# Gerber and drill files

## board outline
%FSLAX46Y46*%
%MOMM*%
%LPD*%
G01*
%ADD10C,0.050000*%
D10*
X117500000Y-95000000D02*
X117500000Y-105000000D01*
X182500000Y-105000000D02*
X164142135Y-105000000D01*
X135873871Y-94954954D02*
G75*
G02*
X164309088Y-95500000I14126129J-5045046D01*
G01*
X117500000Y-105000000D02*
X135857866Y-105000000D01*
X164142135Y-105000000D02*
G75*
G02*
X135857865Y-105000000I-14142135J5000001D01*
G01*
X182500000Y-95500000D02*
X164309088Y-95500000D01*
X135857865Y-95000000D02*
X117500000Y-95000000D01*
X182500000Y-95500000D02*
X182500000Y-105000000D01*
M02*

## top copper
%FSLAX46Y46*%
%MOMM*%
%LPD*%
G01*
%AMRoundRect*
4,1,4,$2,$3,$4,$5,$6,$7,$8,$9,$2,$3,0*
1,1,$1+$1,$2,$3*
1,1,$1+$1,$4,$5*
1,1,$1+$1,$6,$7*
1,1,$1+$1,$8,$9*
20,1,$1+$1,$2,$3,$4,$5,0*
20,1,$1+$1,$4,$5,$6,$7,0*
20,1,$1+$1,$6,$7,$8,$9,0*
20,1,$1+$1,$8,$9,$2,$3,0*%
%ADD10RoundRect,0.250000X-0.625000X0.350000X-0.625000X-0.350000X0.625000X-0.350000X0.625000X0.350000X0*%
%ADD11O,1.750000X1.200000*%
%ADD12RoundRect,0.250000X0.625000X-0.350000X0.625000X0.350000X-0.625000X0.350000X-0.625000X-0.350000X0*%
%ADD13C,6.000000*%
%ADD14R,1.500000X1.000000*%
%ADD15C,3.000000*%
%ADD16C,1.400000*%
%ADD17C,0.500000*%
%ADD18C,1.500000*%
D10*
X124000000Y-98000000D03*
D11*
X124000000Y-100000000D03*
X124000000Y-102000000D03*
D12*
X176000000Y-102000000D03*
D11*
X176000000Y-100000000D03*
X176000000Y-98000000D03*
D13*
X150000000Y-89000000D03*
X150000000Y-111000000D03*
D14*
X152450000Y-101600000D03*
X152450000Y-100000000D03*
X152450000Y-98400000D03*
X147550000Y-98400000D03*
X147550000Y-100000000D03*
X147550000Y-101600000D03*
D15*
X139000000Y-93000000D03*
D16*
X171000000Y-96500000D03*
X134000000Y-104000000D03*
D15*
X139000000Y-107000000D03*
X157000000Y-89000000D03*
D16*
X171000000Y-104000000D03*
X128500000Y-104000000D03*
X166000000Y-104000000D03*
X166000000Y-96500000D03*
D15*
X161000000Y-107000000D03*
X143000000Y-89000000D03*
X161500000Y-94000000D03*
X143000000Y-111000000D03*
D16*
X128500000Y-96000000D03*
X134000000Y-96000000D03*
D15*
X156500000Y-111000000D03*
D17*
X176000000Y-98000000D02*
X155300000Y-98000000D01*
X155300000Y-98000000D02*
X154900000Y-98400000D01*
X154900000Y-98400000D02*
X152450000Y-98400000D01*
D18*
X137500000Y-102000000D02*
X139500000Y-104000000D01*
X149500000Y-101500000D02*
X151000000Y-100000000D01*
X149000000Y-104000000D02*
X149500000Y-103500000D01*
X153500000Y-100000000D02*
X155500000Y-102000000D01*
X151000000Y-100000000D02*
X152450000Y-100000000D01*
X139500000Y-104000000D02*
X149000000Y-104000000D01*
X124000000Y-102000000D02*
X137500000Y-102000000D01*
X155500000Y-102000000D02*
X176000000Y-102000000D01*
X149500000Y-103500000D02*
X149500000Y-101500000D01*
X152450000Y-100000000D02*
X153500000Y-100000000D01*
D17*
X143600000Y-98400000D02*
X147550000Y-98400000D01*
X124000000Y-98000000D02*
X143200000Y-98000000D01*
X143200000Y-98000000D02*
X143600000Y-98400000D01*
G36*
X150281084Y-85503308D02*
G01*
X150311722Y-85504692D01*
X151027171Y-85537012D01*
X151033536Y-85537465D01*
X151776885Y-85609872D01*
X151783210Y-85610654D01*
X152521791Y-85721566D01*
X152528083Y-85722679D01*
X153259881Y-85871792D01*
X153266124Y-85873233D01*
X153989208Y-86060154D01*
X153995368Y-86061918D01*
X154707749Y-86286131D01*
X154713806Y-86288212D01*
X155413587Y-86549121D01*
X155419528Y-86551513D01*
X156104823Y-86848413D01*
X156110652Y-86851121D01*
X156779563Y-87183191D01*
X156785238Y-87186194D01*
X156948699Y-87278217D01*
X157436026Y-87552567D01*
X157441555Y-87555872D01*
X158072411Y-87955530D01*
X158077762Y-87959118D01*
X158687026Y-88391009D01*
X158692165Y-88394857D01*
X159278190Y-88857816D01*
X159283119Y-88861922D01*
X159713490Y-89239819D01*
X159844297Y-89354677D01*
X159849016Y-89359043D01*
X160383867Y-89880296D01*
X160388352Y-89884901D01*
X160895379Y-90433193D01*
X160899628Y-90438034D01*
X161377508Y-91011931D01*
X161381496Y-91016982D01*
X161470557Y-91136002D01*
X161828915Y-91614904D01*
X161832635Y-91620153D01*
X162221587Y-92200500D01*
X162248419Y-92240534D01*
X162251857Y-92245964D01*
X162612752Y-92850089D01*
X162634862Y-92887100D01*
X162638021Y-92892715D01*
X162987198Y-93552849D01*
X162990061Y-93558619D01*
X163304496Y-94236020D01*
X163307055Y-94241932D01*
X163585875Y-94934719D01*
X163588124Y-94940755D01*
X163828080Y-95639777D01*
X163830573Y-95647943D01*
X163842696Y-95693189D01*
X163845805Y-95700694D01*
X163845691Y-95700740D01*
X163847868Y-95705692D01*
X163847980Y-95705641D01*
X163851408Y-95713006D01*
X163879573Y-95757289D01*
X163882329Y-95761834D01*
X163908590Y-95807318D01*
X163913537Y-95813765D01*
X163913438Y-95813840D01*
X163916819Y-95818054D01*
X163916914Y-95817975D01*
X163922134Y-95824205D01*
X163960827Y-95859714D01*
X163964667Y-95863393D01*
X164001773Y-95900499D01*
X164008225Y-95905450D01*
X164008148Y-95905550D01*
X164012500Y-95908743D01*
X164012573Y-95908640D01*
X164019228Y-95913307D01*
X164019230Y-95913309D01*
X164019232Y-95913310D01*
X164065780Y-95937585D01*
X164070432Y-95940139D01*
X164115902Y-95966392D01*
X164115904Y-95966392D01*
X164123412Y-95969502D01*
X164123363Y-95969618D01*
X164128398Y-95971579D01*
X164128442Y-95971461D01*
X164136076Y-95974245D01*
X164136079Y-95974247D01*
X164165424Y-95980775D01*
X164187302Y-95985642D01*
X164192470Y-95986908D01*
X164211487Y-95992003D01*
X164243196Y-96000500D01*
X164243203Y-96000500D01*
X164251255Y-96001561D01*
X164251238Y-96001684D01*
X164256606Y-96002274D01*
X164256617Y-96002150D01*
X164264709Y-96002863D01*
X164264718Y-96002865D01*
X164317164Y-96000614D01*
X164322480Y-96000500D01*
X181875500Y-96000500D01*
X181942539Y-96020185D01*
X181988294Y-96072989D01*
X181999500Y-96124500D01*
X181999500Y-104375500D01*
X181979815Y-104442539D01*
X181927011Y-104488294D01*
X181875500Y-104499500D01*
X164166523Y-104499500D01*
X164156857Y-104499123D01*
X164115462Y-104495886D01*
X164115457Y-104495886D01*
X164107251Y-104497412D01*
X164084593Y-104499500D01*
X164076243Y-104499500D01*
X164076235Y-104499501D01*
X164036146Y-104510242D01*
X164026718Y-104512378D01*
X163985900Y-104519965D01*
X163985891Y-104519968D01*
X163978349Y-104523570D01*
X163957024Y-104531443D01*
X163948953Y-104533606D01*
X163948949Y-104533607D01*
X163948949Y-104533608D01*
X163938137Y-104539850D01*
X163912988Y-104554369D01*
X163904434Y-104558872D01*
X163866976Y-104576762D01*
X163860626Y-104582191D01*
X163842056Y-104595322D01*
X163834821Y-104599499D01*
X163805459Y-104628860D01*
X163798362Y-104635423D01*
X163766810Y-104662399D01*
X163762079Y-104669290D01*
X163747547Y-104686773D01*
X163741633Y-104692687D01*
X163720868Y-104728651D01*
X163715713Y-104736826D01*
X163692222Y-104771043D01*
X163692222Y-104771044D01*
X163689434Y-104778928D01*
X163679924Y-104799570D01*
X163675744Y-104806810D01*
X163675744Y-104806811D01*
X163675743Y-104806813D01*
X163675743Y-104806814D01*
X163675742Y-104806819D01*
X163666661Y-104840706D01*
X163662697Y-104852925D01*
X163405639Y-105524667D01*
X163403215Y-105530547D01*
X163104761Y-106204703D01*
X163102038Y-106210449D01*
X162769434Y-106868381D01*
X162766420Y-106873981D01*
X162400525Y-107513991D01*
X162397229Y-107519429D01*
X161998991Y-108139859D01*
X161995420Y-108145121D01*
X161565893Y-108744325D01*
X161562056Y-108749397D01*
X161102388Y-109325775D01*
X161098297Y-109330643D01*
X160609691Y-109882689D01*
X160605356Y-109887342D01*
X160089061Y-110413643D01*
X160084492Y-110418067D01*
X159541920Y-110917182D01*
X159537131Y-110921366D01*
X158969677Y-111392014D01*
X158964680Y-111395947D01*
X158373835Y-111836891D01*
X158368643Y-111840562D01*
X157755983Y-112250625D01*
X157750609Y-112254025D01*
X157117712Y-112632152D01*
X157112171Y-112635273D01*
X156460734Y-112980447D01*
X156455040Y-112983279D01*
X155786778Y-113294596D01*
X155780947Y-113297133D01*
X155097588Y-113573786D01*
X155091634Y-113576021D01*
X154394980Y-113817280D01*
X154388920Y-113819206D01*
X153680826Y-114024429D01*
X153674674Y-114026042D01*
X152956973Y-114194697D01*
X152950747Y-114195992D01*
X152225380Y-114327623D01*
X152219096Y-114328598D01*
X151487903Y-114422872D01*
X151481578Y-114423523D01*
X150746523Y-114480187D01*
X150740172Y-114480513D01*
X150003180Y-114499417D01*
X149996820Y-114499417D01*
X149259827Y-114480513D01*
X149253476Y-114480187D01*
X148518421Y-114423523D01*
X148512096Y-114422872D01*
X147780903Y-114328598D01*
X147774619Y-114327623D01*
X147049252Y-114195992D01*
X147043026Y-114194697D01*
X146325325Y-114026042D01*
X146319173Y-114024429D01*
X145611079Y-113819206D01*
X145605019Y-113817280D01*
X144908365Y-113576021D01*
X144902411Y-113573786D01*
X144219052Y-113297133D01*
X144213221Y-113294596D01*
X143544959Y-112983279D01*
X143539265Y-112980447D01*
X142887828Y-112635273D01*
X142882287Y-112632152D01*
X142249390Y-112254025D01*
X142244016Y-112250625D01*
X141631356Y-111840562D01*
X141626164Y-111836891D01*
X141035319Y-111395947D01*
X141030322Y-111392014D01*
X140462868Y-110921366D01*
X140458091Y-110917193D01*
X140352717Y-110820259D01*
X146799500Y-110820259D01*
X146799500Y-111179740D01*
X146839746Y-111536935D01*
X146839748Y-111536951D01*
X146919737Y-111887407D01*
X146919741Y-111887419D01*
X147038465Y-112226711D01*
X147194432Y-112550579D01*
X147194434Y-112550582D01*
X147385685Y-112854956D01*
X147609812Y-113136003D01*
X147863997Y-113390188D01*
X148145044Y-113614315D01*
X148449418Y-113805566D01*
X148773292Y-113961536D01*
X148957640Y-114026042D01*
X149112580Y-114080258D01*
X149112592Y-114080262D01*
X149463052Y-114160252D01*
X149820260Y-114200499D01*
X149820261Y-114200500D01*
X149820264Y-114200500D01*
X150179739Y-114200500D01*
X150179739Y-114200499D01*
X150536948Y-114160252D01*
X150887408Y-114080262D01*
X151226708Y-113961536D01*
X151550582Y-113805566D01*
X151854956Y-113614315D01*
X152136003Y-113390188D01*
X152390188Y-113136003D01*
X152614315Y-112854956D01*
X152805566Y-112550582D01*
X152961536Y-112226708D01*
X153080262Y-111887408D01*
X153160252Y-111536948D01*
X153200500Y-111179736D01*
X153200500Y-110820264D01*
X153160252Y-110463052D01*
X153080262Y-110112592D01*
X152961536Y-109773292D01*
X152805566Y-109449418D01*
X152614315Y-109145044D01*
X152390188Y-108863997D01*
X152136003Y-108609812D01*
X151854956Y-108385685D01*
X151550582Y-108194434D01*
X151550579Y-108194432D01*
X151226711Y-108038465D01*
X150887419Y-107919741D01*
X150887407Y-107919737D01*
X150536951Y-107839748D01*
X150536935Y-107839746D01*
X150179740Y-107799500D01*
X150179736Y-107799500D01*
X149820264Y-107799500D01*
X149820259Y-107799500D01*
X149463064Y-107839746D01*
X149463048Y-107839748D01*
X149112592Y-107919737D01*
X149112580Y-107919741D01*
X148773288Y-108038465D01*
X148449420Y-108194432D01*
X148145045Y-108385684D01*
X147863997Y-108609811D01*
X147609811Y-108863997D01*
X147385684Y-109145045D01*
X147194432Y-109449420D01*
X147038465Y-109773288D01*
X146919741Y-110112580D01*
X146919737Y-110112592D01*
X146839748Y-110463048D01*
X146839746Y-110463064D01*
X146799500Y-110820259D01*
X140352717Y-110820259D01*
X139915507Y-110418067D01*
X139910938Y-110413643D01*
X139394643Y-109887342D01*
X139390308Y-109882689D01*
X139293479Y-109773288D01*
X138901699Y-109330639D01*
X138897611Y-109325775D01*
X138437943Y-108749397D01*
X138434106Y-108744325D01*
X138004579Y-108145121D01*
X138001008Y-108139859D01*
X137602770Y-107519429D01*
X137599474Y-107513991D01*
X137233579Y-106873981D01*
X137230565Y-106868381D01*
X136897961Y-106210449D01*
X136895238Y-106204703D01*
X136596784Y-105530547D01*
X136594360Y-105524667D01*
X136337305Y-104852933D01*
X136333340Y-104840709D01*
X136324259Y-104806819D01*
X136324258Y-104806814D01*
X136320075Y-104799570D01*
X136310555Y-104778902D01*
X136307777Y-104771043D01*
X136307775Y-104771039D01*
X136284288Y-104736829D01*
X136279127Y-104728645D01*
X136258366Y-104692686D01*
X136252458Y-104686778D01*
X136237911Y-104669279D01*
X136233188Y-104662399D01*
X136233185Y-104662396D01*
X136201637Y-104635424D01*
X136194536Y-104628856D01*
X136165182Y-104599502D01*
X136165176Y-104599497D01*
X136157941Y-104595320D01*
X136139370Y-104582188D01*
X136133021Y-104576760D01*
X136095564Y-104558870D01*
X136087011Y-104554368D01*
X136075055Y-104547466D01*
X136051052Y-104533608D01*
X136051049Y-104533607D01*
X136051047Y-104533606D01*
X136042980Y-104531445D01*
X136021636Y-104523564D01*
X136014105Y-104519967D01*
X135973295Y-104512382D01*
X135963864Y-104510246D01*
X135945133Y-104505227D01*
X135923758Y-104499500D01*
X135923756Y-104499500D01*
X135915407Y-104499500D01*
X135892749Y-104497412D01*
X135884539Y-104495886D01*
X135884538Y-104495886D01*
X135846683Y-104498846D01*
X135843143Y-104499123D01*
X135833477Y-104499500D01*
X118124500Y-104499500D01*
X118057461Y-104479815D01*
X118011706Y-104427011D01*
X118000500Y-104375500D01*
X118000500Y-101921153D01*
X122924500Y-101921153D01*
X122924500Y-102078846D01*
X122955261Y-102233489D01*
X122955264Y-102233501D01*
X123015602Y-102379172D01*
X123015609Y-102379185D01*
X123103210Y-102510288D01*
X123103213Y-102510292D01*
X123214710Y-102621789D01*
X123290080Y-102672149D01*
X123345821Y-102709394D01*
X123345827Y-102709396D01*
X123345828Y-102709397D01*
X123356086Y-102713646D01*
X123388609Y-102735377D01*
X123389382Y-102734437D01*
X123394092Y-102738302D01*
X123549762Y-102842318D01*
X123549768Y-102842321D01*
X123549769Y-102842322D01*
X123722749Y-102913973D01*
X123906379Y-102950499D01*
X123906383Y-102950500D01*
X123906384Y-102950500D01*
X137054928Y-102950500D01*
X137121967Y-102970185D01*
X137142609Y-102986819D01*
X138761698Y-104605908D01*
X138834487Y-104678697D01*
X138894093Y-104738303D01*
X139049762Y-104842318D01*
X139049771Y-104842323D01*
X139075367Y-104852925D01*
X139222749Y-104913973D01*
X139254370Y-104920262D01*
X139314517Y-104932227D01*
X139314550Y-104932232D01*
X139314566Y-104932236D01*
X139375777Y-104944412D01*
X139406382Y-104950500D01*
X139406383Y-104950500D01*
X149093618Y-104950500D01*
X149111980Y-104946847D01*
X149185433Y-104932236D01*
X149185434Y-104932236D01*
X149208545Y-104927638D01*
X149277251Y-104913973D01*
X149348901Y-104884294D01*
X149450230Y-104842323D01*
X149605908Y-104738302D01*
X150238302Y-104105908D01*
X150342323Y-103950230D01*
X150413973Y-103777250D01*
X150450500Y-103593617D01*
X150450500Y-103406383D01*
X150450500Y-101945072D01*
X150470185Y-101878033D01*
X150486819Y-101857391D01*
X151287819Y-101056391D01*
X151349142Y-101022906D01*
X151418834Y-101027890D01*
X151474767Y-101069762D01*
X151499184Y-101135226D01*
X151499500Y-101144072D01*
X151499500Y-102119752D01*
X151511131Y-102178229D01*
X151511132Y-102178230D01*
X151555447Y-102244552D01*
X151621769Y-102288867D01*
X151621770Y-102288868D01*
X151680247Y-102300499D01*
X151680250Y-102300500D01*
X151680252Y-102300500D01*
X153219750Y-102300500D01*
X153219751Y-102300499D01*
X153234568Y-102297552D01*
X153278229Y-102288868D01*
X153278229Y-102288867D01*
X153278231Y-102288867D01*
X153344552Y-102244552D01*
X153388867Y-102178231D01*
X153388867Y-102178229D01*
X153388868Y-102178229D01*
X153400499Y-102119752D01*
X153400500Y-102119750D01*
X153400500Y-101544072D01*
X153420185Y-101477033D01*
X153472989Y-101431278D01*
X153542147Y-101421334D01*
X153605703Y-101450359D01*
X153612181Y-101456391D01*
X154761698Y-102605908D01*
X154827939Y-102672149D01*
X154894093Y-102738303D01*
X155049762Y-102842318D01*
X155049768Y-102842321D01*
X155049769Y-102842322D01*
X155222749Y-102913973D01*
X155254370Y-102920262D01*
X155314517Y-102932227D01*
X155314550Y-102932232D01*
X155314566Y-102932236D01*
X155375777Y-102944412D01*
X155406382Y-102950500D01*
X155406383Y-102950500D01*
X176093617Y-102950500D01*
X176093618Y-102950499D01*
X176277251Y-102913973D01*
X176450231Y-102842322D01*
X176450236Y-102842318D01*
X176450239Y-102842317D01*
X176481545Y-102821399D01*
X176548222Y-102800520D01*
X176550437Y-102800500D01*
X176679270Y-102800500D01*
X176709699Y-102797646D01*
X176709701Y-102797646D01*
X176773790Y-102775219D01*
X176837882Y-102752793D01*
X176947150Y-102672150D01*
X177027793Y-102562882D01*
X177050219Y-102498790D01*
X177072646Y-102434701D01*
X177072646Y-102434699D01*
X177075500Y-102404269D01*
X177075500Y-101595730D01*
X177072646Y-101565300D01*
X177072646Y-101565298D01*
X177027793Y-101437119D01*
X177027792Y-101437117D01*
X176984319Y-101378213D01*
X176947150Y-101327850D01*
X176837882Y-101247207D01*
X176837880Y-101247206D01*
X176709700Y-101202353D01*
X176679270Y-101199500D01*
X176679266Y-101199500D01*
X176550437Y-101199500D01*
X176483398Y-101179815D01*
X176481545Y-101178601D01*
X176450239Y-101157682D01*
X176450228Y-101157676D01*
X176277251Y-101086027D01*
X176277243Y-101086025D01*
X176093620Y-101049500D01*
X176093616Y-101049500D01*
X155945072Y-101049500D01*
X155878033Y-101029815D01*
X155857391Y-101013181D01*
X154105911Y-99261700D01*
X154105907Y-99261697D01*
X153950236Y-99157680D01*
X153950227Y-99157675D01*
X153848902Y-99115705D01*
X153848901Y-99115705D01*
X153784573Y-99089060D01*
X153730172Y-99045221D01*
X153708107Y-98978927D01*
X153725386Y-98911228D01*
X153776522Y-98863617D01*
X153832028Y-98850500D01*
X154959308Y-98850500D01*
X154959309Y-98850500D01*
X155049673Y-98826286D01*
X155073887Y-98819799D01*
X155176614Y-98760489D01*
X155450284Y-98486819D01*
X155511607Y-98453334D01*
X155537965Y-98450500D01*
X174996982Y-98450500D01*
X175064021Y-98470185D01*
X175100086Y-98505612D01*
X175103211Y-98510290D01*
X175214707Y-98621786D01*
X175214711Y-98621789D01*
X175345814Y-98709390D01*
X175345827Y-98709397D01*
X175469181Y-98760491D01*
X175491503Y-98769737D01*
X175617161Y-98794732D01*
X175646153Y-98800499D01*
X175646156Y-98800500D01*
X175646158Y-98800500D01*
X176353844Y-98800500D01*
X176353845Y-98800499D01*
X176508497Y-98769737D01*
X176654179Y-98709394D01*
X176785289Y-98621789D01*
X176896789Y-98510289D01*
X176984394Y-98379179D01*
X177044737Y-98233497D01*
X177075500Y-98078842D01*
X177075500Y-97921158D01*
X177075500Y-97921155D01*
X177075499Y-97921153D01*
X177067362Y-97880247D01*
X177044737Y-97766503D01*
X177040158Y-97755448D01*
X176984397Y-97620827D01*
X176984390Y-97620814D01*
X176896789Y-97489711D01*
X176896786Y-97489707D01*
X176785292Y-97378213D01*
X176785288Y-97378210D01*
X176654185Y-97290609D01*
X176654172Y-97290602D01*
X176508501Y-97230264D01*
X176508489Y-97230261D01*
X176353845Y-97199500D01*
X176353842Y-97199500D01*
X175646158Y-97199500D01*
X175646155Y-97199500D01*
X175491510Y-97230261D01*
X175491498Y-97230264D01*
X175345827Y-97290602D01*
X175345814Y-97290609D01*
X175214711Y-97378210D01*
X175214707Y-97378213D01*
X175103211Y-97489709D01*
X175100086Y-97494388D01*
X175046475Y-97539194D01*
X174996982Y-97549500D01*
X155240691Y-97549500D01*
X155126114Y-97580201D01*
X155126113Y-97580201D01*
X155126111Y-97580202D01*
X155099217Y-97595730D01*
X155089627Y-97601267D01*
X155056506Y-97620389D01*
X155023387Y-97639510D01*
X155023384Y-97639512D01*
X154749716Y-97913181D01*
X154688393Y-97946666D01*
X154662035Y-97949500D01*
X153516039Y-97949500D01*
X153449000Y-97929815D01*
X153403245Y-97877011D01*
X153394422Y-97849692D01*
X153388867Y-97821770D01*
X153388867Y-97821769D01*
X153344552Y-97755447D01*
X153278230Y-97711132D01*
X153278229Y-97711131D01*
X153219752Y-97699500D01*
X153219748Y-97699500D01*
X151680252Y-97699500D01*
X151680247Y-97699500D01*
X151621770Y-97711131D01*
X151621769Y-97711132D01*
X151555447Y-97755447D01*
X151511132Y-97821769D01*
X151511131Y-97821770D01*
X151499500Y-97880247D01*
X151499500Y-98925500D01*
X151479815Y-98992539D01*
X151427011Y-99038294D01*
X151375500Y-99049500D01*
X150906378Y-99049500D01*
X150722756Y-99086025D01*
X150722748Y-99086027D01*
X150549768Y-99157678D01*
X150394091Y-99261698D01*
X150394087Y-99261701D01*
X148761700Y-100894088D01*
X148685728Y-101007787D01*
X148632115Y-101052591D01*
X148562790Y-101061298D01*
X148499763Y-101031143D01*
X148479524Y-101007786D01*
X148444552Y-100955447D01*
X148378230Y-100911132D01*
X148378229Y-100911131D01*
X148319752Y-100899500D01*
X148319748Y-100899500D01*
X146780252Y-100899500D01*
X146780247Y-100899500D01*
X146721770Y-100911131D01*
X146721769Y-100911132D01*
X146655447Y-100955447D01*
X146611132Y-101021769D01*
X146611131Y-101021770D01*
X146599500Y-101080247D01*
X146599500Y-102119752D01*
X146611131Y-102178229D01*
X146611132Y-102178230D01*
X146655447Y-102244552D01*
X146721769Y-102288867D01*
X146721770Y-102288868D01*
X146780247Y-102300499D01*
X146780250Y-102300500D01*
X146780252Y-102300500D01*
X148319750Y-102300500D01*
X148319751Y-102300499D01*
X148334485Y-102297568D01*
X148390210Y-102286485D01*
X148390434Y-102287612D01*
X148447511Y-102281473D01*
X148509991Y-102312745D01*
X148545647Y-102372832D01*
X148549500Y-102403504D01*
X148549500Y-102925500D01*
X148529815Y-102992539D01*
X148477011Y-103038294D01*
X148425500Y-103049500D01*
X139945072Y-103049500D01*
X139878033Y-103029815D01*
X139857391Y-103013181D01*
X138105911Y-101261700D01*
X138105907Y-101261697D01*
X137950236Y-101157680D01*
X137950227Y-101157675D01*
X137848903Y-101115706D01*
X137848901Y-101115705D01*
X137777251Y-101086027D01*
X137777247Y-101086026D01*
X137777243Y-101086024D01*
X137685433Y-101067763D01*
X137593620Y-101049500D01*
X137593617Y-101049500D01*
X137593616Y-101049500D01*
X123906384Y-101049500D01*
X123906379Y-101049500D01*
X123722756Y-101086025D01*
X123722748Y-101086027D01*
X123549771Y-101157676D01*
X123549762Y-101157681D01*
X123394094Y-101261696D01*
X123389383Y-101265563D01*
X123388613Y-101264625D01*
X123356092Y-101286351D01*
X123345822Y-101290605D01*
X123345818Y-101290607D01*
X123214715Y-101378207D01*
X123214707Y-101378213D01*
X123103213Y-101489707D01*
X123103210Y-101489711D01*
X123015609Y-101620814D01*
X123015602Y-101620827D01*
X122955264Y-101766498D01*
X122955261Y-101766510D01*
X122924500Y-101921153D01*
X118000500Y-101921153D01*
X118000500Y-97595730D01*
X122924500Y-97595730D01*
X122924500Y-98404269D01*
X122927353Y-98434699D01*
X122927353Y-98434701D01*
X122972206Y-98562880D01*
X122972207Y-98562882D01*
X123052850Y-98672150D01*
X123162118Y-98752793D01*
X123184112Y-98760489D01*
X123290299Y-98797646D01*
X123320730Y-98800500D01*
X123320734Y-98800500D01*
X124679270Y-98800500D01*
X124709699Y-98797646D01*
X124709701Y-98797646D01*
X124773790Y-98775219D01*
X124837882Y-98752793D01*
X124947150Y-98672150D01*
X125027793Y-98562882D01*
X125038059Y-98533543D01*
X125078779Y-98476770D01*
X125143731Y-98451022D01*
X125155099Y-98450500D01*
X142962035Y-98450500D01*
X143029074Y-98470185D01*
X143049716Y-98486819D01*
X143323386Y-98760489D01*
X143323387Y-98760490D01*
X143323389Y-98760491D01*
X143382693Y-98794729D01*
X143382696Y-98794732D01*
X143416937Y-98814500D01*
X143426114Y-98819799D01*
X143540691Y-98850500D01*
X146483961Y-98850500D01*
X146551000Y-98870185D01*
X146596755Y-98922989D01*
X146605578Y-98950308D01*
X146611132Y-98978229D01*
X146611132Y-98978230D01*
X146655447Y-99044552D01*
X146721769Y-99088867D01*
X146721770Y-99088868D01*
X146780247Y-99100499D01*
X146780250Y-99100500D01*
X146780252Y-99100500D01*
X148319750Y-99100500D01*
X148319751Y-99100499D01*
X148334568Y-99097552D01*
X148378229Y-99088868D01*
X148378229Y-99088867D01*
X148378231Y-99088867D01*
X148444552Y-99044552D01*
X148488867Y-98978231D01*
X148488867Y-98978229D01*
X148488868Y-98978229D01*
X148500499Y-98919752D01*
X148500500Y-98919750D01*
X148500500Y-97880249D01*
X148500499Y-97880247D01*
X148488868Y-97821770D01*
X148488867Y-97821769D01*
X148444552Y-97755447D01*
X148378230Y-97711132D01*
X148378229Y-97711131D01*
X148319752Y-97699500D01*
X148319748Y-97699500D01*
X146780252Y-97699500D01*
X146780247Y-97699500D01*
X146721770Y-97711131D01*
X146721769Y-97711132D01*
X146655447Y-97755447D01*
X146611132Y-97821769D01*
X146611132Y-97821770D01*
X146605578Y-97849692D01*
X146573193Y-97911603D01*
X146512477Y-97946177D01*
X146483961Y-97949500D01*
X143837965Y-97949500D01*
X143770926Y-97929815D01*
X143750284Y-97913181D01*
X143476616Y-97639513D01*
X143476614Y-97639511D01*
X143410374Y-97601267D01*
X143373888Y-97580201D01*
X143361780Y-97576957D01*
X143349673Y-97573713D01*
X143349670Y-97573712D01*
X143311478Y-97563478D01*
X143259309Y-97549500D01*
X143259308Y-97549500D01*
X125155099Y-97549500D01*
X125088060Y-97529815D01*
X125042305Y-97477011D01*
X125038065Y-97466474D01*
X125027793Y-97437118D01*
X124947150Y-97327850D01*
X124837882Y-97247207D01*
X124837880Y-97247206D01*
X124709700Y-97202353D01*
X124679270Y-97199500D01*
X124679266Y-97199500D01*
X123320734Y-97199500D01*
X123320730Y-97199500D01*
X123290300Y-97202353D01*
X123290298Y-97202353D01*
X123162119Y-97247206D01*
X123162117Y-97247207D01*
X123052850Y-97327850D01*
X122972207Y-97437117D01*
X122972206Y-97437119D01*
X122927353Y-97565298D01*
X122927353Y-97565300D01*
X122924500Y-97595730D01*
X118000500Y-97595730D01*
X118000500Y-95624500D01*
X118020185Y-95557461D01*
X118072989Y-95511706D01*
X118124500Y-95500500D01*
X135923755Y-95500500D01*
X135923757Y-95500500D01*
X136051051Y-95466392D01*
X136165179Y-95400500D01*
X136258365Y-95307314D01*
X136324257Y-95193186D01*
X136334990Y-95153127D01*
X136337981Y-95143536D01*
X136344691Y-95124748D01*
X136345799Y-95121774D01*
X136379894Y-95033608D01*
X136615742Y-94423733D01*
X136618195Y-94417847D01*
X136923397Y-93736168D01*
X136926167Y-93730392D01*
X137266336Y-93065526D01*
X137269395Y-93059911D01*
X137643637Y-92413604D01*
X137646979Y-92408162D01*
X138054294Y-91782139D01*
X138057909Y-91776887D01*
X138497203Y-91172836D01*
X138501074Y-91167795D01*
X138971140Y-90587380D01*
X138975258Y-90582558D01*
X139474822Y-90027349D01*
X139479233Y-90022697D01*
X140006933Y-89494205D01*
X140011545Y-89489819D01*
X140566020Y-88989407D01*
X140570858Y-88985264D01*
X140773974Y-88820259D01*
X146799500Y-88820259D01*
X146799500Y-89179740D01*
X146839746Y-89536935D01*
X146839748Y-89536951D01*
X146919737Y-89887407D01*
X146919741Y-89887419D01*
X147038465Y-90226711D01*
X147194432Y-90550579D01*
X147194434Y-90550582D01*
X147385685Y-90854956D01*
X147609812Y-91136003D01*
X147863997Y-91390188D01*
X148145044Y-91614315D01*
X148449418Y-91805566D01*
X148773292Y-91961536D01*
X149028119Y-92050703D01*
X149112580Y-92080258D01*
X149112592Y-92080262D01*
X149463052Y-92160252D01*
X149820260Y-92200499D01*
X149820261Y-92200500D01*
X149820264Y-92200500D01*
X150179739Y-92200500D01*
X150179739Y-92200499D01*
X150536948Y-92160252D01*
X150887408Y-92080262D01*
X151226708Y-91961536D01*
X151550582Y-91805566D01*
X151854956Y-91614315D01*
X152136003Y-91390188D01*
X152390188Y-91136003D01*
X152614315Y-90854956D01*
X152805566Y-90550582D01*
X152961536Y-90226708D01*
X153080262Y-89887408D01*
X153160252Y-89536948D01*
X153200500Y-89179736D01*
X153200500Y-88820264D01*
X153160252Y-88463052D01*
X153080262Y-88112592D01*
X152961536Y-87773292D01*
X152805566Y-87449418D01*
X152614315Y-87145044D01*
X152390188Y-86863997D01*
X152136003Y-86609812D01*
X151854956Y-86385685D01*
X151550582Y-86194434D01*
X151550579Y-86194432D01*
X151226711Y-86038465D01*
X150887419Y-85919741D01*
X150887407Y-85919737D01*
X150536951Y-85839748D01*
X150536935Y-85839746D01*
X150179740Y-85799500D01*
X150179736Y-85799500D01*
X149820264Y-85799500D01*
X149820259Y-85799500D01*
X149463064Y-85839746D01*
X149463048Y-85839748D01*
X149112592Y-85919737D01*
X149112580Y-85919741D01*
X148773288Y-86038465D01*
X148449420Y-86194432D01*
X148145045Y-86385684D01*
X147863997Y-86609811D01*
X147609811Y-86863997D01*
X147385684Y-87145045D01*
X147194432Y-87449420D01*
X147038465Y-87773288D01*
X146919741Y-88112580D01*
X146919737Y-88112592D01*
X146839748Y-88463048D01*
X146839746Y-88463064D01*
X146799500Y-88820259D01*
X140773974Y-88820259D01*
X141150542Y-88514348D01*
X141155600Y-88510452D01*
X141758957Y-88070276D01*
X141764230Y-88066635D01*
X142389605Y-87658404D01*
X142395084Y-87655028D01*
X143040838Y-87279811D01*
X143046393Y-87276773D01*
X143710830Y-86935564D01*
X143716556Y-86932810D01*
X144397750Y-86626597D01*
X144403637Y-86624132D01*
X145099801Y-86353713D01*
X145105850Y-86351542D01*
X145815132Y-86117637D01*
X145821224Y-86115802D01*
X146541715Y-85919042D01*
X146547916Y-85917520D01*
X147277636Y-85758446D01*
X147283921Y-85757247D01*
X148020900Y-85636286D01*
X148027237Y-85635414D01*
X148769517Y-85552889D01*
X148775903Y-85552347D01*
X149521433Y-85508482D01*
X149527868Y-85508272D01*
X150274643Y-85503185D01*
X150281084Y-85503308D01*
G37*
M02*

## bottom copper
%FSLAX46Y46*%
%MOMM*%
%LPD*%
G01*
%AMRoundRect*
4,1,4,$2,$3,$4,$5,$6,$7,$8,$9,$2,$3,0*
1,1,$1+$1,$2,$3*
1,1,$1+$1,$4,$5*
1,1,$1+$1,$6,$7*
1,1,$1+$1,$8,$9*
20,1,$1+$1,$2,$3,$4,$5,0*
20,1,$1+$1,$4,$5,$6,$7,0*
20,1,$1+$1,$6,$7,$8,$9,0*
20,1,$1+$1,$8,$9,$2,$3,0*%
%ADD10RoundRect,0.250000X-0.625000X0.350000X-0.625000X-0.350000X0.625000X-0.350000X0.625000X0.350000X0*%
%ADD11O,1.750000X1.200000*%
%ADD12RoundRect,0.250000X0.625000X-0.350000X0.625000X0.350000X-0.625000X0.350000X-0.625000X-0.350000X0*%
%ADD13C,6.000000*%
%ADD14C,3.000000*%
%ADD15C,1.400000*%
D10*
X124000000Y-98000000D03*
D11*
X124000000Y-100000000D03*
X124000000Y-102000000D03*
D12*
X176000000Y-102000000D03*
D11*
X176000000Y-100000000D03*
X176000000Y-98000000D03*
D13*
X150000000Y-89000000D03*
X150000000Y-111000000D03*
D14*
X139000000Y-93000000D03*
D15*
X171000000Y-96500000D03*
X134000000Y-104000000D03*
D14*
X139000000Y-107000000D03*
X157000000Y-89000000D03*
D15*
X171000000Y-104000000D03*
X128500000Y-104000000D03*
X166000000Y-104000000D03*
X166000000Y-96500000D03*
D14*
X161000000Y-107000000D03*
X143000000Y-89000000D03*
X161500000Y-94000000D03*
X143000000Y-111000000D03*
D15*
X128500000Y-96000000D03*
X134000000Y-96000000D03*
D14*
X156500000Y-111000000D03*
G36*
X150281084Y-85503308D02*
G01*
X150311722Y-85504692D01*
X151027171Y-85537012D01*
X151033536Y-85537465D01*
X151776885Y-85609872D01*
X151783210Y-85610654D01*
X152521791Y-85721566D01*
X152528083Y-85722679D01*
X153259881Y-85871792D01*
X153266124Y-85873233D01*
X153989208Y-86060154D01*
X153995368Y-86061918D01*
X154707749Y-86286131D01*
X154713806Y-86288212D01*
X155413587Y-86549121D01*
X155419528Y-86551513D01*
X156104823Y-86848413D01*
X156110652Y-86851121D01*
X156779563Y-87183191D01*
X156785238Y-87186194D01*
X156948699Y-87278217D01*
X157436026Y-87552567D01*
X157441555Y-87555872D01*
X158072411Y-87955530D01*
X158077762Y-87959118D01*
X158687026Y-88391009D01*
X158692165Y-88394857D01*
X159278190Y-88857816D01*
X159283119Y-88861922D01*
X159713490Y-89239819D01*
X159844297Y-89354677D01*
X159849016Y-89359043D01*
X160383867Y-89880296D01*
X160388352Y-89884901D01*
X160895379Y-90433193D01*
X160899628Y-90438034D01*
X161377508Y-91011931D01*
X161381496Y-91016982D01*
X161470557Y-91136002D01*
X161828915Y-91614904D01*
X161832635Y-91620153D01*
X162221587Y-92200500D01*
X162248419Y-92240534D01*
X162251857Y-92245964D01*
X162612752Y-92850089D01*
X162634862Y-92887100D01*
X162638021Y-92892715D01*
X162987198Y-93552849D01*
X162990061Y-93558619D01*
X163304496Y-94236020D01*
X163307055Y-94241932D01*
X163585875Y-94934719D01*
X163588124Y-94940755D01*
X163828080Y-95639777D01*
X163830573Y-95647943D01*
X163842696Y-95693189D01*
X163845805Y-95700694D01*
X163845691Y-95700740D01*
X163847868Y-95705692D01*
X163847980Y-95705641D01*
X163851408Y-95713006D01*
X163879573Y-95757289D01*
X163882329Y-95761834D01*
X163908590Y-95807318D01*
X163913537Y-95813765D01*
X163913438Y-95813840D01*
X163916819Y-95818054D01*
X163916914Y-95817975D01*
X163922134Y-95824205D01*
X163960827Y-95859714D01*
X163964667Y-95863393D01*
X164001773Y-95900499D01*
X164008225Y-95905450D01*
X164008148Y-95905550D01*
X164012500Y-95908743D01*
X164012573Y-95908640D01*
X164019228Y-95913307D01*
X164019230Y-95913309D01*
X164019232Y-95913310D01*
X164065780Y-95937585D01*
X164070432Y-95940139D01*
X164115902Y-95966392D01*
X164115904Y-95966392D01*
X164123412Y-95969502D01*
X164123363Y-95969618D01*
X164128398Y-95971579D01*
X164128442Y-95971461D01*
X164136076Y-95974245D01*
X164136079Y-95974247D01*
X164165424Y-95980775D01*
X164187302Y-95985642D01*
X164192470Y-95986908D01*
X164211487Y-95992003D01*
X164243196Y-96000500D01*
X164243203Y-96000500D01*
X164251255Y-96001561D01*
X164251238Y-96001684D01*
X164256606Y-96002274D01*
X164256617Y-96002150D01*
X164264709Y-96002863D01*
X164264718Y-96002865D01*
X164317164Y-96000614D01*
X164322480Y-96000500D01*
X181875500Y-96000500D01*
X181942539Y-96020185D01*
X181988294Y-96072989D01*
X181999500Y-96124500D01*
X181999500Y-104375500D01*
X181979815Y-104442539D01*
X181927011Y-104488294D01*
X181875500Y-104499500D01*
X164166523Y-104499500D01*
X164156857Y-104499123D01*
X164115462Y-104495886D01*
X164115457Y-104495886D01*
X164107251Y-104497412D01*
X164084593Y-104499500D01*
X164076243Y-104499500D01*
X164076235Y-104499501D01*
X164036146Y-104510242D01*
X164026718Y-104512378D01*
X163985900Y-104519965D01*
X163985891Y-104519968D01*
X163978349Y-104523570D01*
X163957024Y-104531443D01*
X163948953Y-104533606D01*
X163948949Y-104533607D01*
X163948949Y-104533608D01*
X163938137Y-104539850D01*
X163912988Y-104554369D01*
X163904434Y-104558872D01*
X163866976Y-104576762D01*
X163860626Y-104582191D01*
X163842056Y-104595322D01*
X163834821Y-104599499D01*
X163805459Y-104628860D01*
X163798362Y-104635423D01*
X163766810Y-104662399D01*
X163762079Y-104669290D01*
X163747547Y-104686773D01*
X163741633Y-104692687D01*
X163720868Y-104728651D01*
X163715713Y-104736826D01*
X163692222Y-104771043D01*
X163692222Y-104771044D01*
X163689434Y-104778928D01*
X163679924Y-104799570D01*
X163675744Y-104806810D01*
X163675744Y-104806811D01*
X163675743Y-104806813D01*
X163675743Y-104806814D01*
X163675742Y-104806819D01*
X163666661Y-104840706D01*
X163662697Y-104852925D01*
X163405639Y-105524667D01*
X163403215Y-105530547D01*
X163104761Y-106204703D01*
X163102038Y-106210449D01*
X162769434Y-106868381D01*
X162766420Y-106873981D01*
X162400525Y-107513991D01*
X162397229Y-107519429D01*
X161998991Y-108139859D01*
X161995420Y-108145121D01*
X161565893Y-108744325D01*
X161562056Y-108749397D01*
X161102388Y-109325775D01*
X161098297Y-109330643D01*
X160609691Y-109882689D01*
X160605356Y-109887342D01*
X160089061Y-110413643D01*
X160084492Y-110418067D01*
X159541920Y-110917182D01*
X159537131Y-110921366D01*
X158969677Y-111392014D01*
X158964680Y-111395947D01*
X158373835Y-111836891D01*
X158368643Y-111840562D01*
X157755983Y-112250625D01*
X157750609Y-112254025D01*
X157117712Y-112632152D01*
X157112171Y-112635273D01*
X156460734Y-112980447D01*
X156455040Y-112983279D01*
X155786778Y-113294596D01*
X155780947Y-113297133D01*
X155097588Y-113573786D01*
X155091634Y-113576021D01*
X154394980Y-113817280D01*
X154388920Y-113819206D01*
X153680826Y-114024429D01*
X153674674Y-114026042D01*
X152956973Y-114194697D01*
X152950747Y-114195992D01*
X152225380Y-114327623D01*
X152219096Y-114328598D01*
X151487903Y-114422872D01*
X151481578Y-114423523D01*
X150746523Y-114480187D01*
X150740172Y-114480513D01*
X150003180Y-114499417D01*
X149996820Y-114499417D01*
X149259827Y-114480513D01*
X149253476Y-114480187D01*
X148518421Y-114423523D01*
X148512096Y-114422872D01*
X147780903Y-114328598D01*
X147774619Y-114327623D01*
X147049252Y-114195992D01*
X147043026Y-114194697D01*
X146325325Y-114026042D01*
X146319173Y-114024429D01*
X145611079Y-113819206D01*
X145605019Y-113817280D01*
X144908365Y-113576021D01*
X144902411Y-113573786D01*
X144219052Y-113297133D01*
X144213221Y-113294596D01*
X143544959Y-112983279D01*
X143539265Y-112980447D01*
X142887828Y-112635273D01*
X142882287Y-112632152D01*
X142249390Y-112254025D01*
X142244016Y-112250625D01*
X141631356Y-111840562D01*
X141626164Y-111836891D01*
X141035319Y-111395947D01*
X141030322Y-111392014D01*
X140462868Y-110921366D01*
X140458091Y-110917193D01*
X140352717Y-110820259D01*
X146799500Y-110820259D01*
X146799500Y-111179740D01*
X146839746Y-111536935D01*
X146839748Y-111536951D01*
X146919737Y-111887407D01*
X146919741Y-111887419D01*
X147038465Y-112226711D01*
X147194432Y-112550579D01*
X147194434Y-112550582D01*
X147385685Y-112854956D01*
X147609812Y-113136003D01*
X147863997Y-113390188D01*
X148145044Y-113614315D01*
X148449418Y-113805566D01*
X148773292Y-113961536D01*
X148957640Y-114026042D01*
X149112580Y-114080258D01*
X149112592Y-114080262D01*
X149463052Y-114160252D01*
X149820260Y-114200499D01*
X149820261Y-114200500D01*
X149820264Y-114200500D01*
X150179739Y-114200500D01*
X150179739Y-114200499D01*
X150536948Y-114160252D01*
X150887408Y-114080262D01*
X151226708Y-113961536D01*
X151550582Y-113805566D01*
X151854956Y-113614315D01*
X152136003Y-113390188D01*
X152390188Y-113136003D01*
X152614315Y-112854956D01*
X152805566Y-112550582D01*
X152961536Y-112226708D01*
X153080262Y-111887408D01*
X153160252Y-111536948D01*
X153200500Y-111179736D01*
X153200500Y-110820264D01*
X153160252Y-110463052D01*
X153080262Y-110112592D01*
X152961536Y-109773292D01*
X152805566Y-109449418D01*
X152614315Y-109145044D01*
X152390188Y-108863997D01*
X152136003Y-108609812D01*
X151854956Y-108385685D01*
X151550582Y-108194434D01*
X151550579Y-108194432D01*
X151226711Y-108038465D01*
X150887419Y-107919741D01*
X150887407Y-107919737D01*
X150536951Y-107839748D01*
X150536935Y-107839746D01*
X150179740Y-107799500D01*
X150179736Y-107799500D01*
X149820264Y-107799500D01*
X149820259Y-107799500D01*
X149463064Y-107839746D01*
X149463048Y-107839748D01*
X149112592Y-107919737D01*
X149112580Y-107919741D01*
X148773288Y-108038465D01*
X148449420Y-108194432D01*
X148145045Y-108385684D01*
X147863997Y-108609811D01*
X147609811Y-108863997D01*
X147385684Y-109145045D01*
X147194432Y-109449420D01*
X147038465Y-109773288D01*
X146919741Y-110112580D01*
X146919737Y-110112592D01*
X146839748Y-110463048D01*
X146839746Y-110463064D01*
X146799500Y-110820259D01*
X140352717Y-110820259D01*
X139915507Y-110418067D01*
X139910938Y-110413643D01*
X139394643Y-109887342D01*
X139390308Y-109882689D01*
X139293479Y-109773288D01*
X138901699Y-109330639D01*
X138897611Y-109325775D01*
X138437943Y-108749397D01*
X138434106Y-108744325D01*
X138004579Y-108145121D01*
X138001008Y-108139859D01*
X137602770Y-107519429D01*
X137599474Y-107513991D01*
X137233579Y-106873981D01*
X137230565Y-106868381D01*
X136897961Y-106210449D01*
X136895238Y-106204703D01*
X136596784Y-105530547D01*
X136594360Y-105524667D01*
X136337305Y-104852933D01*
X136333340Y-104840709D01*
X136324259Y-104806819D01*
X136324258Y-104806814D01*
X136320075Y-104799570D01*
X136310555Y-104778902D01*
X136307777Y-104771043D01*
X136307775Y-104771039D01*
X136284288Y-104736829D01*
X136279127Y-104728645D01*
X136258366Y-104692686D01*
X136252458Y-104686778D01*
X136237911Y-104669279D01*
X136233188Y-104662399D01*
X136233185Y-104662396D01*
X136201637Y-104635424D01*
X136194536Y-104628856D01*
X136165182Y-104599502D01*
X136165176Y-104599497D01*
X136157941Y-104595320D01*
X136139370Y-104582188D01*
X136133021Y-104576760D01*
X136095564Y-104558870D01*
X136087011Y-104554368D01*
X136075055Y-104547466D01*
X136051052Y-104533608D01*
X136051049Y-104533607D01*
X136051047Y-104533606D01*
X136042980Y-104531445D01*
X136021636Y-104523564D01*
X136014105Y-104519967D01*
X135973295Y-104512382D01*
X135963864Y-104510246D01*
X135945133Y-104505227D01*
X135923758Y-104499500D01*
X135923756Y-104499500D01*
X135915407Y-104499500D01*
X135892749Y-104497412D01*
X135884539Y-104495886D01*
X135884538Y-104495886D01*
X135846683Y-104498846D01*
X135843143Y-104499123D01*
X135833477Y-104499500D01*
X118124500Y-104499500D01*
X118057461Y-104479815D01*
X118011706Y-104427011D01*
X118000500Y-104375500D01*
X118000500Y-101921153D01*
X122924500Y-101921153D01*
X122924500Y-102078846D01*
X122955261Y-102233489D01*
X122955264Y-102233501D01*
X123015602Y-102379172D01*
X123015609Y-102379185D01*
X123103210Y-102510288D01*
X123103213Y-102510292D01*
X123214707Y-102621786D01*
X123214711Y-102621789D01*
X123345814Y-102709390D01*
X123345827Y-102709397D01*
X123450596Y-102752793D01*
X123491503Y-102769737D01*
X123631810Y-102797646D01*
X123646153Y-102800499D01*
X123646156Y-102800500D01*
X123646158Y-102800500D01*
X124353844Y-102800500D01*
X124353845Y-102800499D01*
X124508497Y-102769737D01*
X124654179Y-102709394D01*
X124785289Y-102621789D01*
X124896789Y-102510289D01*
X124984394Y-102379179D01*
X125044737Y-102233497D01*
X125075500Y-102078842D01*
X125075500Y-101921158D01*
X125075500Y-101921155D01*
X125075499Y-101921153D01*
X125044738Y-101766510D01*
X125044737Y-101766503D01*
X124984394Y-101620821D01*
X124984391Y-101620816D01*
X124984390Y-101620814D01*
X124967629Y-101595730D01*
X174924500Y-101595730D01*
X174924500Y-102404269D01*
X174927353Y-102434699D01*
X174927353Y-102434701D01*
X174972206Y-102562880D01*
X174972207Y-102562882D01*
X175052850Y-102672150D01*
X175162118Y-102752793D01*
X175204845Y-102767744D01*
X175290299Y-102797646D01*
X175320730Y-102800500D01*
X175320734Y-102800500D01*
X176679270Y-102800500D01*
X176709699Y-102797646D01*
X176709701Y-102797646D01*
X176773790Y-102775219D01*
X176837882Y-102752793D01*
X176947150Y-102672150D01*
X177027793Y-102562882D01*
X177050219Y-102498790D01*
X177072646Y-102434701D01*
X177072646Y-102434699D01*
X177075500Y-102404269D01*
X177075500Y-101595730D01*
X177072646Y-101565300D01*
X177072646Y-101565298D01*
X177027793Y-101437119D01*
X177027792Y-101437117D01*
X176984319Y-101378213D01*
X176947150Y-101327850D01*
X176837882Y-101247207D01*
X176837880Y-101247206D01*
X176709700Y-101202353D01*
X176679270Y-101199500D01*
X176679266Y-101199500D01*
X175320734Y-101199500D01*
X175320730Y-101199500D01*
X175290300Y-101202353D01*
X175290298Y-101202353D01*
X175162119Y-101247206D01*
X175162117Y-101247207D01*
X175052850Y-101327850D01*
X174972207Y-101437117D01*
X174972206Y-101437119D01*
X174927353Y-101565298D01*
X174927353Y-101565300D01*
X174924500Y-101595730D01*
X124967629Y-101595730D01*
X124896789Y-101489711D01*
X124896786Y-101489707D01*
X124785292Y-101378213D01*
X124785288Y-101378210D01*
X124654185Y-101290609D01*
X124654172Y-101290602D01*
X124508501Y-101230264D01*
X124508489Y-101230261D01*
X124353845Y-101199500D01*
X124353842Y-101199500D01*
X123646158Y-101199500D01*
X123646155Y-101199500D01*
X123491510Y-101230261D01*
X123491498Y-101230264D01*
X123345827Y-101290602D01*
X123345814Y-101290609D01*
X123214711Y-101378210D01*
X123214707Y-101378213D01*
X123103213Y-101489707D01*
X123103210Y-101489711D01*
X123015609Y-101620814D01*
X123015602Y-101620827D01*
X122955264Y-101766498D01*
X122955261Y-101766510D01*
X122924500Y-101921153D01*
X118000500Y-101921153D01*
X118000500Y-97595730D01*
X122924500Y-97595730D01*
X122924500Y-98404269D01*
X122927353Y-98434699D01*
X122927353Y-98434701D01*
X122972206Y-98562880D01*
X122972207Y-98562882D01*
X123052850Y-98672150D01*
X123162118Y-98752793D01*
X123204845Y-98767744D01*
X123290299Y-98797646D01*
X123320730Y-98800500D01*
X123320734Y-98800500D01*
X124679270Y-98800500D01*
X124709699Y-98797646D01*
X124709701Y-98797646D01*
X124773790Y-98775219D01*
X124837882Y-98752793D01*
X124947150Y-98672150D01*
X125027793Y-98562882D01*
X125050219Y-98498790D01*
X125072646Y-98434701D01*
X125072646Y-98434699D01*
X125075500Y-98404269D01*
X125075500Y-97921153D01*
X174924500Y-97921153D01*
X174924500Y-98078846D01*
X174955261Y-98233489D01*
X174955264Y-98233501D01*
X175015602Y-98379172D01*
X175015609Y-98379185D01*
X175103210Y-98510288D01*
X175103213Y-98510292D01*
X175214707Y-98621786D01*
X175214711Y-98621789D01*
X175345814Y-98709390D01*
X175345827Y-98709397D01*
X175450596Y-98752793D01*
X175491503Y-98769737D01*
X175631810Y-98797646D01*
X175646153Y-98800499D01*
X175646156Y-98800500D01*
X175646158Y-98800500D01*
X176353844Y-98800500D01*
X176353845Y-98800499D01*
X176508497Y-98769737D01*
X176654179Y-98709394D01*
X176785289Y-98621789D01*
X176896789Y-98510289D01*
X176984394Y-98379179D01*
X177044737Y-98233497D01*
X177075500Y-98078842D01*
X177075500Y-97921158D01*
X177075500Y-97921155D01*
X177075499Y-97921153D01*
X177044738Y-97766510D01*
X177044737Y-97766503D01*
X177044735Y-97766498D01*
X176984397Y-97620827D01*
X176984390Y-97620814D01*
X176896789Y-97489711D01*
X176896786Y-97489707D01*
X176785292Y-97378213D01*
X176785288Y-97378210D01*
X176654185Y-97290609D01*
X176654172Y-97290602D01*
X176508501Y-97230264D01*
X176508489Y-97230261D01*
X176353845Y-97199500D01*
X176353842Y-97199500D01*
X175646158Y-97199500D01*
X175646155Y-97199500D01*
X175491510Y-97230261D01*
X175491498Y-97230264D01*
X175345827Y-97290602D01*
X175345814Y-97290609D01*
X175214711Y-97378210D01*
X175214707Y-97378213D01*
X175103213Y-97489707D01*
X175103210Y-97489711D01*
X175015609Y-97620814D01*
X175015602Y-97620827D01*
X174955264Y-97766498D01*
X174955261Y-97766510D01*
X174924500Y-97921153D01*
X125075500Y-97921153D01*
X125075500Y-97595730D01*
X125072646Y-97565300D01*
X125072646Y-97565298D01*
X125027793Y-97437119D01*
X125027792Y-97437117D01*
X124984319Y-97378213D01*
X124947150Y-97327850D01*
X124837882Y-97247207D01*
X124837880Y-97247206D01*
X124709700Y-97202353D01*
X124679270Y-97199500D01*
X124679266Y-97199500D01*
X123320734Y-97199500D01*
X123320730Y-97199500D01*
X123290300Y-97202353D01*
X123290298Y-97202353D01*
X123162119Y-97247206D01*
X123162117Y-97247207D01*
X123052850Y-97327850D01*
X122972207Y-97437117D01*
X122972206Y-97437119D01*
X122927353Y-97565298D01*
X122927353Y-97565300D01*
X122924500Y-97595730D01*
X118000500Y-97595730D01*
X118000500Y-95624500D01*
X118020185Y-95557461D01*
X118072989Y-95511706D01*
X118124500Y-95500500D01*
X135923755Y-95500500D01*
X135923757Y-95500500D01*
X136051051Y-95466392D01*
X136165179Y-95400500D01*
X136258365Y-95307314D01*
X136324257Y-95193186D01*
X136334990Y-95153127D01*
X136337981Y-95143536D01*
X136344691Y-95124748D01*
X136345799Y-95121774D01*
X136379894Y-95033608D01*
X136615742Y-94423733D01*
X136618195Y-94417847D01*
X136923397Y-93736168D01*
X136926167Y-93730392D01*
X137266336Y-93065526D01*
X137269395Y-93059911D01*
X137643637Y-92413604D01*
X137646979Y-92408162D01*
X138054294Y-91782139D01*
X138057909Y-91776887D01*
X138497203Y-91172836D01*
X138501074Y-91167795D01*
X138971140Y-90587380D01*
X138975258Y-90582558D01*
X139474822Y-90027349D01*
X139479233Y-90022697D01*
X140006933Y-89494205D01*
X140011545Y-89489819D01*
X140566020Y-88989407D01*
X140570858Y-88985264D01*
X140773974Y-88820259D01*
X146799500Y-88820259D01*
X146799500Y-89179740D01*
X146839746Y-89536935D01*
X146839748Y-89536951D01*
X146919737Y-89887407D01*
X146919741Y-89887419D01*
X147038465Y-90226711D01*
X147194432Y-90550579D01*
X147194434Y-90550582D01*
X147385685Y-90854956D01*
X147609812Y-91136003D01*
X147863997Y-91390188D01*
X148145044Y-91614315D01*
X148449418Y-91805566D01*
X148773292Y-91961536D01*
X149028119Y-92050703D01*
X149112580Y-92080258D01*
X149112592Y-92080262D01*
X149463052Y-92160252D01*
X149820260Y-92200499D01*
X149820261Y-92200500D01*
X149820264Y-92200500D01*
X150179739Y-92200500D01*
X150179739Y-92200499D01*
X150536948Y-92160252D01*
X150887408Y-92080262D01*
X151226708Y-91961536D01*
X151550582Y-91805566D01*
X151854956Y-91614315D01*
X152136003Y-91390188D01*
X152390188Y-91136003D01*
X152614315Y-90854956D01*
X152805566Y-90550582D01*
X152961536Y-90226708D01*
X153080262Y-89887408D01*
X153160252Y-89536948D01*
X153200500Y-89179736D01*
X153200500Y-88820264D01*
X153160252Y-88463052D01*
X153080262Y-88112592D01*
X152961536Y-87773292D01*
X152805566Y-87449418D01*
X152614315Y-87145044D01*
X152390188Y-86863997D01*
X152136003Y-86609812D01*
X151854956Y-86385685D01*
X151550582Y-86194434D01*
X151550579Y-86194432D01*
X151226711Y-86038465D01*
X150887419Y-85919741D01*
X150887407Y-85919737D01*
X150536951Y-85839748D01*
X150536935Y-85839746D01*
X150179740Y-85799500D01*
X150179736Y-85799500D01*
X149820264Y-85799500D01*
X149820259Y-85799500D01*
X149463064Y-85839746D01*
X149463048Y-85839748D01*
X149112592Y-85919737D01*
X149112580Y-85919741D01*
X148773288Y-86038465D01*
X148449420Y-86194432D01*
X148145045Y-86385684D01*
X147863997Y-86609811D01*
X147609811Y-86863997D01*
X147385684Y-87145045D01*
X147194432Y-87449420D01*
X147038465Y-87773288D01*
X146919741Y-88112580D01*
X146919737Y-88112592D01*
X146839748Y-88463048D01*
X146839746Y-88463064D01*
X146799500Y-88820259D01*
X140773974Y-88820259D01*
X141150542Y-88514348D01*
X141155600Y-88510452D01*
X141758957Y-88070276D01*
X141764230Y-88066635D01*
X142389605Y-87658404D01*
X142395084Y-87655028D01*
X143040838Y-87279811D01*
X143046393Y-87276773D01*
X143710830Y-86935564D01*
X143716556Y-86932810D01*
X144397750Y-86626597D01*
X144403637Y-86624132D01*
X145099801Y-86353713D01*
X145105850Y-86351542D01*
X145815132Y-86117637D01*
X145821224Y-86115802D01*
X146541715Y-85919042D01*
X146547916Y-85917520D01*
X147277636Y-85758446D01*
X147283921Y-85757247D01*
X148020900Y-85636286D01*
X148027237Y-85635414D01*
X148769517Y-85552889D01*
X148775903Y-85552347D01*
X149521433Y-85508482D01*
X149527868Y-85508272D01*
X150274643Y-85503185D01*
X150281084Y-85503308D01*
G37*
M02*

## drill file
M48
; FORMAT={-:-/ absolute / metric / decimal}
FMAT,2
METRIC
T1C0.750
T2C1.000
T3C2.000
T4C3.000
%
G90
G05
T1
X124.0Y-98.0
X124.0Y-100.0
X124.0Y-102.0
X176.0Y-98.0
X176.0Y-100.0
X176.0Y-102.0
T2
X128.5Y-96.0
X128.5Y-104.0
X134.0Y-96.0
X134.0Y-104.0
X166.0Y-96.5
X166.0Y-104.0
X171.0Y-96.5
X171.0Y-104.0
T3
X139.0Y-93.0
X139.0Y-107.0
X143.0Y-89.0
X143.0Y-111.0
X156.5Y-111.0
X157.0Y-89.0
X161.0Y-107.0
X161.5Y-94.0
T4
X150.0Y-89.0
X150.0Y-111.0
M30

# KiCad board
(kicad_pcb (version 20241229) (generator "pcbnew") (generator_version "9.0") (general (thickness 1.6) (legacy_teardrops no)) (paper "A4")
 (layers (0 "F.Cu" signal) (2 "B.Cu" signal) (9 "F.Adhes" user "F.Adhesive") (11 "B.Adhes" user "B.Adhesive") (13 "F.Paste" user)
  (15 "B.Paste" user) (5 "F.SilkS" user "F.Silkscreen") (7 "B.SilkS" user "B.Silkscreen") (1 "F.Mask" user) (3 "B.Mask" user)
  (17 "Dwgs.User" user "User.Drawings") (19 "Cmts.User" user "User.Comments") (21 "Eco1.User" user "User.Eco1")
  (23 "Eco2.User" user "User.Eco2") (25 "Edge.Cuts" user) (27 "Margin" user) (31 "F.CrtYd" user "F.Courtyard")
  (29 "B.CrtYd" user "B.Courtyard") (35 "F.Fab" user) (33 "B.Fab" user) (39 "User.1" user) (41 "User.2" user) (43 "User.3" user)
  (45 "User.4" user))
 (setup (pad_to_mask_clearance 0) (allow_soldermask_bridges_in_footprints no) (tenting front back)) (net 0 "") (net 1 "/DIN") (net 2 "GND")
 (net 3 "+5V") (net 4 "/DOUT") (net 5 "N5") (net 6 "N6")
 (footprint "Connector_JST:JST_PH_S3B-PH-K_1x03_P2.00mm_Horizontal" (layer "F.Cu") (at 124 98 -90)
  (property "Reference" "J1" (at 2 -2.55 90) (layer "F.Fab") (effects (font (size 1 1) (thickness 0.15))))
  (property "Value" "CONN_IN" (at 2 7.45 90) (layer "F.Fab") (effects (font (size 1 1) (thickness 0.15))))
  (pad "1" thru_hole roundrect (at 0 0 270) (size 1.2 1.75) (drill 0.75) (layers "*.Cu" "*.Mask") (remove_unused_layers no)
   (roundrect_rratio 0.208333) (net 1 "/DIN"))
  (pad "2" thru_hole oval (at 2 0 270) (size 1.2 1.75) (drill 0.75) (layers "*.Cu" "*.Mask") (remove_unused_layers no) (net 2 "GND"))
  (pad "3" thru_hole oval (at 4 0 270) (size 1.2 1.75) (drill 0.75) (layers "*.Cu" "*.Mask") (remove_unused_layers no) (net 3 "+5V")))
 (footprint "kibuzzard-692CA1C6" (layer "F.Cu") (at 127 100 -90)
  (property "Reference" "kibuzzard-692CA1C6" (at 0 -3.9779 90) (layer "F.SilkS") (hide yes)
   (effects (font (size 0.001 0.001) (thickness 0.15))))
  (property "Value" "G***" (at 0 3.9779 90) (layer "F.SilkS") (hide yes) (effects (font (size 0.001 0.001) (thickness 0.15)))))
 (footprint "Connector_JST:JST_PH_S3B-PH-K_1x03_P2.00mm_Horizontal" (layer "F.Cu") (at 176 102 90)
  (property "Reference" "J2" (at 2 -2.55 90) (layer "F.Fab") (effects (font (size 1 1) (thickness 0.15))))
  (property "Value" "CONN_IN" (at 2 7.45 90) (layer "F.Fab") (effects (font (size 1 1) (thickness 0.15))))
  (pad "1" thru_hole roundrect (at 0 0 90) (size 1.2 1.75) (drill 0.75) (layers "*.Cu" "*.Mask") (remove_unused_layers no)
   (roundrect_rratio 0.208333) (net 3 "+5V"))
  (pad "2" thru_hole oval (at 2 0 90) (size 1.2 1.75) (drill 0.75) (layers "*.Cu" "*.Mask") (remove_unused_layers no) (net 2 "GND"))
  (pad "3" thru_hole oval (at 4 0 90) (size 1.2 1.75) (drill 0.75) (layers "*.Cu" "*.Mask") (remove_unused_layers no) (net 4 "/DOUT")))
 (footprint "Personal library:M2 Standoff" (layer "F.Cu") (at 150 89 180)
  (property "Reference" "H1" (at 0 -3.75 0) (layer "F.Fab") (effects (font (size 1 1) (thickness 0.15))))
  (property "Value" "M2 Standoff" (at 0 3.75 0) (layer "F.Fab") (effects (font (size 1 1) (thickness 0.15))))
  (pad "1" thru_hole circle (at 0 0 180) (size 6 6) (drill 3) (layers "*.Cu" "*.Mask") (remove_unused_layers no) (zone_connect 2)))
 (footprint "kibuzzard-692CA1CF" (layer "F.Cu") (at 173 100 90)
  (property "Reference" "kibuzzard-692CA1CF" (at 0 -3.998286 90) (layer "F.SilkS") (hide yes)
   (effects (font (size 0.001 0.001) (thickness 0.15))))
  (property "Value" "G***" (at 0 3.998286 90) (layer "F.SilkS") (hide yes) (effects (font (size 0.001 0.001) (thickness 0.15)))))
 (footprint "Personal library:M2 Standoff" (layer "F.Cu") (at 150 111 180)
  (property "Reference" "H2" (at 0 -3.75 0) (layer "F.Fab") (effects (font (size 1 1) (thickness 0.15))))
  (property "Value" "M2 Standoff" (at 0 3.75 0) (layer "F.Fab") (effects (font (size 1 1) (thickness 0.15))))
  (pad "1" thru_hole circle (at 0 0 180) (size 6 6) (drill 3) (layers "*.Cu" "*.Mask") (remove_unused_layers no) (zone_connect 2)))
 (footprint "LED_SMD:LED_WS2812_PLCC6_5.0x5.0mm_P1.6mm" (layer "F.Cu") (at 150 100 180)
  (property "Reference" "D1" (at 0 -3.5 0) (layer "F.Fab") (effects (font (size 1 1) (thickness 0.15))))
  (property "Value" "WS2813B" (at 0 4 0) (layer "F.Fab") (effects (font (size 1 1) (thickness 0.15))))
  (pad "1" smd rect (at -2.45 -1.6 180) (size 1.5 1) (layers "F.Cu" "F.Mask" "F.Paste") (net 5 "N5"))
  (pad "2" smd rect (at -2.45 0 180) (size 1.5 1) (layers "F.Cu" "F.Mask" "F.Paste") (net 3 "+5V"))
  (pad "3" smd rect (at -2.45 1.6 180) (size 1.5 1) (layers "F.Cu" "F.Mask" "F.Paste") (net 4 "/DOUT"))
  (pad "4" smd rect (at 2.45 1.6 180) (size 1.5 1) (layers "F.Cu" "F.Mask" "F.Paste") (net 1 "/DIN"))
  (pad "5" smd rect (at 2.45 0 180) (size 1.5 1) (layers "F.Cu" "F.Mask" "F.Paste") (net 2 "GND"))
  (pad "6" smd rect (at 2.45 -1.6 180) (size 1.5 1) (layers "F.Cu" "F.Mask" "F.Paste") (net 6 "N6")))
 (gr_line (start 117.5 95) (end 117.5 105) (stroke (width 0.05) (type default)) (layer "Edge.Cuts"))
 (gr_line (start 182.5 105) (end 164.142135 105) (stroke (width 0.05) (type default)) (layer "Edge.Cuts"))
 (gr_arc (start 135.873871 94.954954) (mid 150.287467 85.002755) (end 164.309088 95.5) (stroke (width 0.05) (type default))
  (layer "Edge.Cuts"))
 (gr_line (start 117.5 105) (end 135.857866 105) (stroke (width 0.05) (type default)) (layer "Edge.Cuts"))
 (gr_arc (start 164.142135 105) (mid 150 114.999999) (end 135.857865 105) (stroke (width 0.05) (type default)) (layer "Edge.Cuts"))
 (gr_line (start 182.5 95.5) (end 164.309088 95.5) (stroke (width 0.05) (type default)) (layer "Edge.Cuts"))
 (gr_line (start 135.857865 95) (end 117.5 95) (stroke (width 0.05) (type default)) (layer "Edge.Cuts"))
 (gr_line (start 182.5 95.5) (end 182.5 105) (stroke (width 0.05) (type default)) (layer "Edge.Cuts"))
 (segment (start 176 98) (end 155.3 98) (width 0.5) (layer "F.Cu") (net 4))
 (segment (start 155.3 98) (end 154.9 98.4) (width 0.5) (layer "F.Cu") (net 4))
 (segment (start 154.9 98.4) (end 152.45 98.4) (width 0.5) (layer "F.Cu") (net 4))
 (via (at 139 93) (size 3) (drill 2) (layers "F.Cu" "B.Cu") (free yes) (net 2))
 (via (at 171 96.5) (size 1.4) (drill 1) (layers "F.Cu" "B.Cu") (free yes) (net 2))
 (via (at 134 104) (size 1.4) (drill 1) (layers "F.Cu" "B.Cu") (free yes) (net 2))
 (via (at 139 107) (size 3) (drill 2) (layers "F.Cu" "B.Cu") (free yes) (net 2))
 (via (at 157 89) (size 3) (drill 2) (layers "F.Cu" "B.Cu") (free yes) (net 2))
 (via (at 171 104) (size 1.4) (drill 1) (layers "F.Cu" "B.Cu") (free yes) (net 2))
 (via (at 128.5 104) (size 1.4) (drill 1) (layers "F.Cu" "B.Cu") (free yes) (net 2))
 (via (at 166 104) (size 1.4) (drill 1) (layers "F.Cu" "B.Cu") (free yes) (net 2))
 (via (at 166 96.5) (size 1.4) (drill 1) (layers "F.Cu" "B.Cu") (free yes) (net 2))
 (via (at 161 107) (size 3) (drill 2) (layers "F.Cu" "B.Cu") (free yes) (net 2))
 (via (at 143 89) (size 3) (drill 2) (layers "F.Cu" "B.Cu") (free yes) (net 2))
 (via (at 161.5 94) (size 3) (drill 2) (layers "F.Cu" "B.Cu") (free yes) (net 2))
 (via (at 143 111) (size 3) (drill 2) (layers "F.Cu" "B.Cu") (free yes) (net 2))
 (via (at 128.5 96) (size 1.4) (drill 1) (layers "F.Cu" "B.Cu") (free yes) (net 2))
 (via (at 134 96) (size 1.4) (drill 1) (layers "F.Cu" "B.Cu") (free yes) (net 2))
 (via (at 156.5 111) (size 3) (drill 2) (layers "F.Cu" "B.Cu") (free yes) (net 2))
 (segment (start 137.5 102) (end 139.5 104) (width 1.5) (layer "F.Cu") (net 3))
 (segment (start 149.5 101.5) (end 151 100) (width 1.5) (layer "F.Cu") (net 3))
 (segment (start 149 104) (end 149.5 103.5) (width 1.5) (layer "F.Cu") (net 3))
 (segment (start 153.5 100) (end 155.5 102) (width 1.5) (layer "F.Cu") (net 3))
 (segment (start 151 100) (end 152.45 100) (width 1.5) (layer "F.Cu") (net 3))
 (segment (start 139.5 104) (end 149 104) (width 1.5) (layer "F.Cu") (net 3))
 (segment (start 124 102) (end 137.5 102) (width 1.5) (layer "F.Cu") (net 3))
 (segment (start 155.5 102) (end 176 102) (width 1.5) (layer "F.Cu") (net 3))
 (segment (start 149.5 103.5) (end 149.5 101.5) (width 1.5) (layer "F.Cu") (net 3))
 (segment (start 152.45 100) (end 153.5 100) (width 1.5) (layer "F.Cu") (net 3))
 (segment (start 143.6 98.4) (end 147.55 98.4) (width 0.5) (layer "F.Cu") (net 1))
 (segment (start 124 98) (end 143.2 98) (width 0.5) (layer "F.Cu") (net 1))
 (segment (start 143.2 98) (end 143.6 98.4) (width 0.5) (layer "F.Cu") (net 1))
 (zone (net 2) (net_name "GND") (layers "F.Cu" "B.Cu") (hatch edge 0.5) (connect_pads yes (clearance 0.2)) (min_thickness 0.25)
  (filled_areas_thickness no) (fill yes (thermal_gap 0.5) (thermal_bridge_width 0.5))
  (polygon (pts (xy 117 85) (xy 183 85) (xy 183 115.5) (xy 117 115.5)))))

